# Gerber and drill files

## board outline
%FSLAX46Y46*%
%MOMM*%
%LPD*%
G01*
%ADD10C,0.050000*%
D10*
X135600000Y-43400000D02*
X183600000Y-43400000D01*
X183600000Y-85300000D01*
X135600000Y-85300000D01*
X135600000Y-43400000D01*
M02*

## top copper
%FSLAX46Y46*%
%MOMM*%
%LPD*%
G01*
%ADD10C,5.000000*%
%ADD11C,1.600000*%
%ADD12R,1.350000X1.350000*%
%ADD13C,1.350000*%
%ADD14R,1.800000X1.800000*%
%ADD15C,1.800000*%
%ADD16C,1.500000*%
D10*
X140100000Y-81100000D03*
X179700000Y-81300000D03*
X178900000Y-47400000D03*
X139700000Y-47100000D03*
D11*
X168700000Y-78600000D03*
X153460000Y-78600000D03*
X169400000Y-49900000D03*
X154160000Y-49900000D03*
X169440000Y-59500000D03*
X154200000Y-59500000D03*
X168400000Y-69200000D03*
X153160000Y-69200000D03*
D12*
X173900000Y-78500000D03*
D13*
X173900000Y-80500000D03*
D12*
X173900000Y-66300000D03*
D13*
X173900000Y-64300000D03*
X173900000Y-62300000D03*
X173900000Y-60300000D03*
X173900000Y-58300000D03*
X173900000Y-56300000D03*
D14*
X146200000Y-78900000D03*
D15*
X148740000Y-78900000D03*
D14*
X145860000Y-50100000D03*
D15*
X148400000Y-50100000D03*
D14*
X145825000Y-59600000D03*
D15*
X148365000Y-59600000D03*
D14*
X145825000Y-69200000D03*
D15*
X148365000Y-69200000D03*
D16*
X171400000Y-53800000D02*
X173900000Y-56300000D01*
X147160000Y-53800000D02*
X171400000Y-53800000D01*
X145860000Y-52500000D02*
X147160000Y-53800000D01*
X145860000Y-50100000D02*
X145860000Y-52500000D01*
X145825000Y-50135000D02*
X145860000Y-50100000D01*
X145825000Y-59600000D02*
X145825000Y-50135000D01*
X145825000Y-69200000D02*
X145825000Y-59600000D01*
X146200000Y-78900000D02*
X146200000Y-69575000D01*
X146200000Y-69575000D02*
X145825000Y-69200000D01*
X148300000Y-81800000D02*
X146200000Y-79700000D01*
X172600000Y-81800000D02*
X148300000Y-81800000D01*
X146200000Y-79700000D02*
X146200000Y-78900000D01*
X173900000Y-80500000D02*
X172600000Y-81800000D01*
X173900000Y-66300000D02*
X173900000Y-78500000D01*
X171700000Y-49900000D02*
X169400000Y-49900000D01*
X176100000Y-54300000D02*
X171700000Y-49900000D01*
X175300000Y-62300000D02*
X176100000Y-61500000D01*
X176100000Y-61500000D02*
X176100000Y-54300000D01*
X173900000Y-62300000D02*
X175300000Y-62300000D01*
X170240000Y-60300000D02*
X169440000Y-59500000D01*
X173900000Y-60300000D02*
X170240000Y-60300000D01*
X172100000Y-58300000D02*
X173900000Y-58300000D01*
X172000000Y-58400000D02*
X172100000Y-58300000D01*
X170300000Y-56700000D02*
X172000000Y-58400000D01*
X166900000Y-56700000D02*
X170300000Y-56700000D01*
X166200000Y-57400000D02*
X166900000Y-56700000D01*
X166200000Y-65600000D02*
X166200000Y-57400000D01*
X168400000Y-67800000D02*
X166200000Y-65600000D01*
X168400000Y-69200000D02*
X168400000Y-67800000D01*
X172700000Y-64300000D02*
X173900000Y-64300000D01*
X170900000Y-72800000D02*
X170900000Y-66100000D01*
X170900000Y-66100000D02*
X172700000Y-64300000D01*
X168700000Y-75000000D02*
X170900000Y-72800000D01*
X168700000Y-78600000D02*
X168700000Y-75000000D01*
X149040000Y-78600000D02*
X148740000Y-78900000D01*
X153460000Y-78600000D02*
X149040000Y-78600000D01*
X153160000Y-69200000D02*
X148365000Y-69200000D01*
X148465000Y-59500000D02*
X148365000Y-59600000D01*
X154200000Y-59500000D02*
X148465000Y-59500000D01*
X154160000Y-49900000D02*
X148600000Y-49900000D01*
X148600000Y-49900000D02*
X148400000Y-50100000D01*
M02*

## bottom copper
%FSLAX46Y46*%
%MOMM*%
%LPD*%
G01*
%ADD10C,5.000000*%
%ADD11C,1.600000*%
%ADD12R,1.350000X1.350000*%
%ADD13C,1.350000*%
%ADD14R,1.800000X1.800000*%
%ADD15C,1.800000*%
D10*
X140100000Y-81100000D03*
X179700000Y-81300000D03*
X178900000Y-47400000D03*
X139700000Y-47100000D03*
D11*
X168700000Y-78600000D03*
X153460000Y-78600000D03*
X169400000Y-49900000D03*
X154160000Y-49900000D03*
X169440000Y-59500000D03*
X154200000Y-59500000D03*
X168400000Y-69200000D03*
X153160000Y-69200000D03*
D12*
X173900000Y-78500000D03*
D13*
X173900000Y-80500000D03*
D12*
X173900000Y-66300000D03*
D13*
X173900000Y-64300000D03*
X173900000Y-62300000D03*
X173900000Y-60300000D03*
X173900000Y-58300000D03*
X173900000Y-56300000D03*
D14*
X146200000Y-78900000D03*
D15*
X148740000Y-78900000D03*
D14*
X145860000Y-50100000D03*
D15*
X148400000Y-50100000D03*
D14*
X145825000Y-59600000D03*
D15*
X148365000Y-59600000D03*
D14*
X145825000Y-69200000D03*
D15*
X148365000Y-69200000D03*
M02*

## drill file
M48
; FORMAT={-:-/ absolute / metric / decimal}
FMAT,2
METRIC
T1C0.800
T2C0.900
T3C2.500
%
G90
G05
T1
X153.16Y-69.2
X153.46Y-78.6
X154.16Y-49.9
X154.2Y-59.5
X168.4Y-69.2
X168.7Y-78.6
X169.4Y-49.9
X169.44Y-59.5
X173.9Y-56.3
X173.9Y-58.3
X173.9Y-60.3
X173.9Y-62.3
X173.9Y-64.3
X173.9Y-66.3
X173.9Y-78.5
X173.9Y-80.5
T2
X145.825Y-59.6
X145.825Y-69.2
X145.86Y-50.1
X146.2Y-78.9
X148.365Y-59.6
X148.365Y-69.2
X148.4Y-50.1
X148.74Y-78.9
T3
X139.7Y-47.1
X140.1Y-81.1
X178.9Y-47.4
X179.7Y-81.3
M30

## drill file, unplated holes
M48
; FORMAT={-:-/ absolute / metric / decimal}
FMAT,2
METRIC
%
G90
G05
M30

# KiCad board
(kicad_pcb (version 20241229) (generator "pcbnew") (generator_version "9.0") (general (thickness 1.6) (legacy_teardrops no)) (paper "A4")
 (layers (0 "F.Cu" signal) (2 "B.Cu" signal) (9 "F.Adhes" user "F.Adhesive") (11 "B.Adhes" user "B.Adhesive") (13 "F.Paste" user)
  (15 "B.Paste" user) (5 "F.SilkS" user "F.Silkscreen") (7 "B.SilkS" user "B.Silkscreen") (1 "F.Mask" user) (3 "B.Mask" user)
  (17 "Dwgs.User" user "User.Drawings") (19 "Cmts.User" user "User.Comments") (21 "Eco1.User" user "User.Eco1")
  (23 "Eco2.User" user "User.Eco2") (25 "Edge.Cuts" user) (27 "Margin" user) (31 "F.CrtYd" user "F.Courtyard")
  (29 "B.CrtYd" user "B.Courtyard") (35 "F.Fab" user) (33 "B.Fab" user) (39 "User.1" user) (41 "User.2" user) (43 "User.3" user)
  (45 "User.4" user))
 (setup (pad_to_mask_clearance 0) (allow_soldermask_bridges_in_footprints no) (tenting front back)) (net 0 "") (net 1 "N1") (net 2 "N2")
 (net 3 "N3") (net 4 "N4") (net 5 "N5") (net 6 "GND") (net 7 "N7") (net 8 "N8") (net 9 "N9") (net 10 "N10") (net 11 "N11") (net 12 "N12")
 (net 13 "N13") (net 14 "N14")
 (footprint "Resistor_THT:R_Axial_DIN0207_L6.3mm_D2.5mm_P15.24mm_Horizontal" (layer "F.Cu") (at 169.44 59.5 180)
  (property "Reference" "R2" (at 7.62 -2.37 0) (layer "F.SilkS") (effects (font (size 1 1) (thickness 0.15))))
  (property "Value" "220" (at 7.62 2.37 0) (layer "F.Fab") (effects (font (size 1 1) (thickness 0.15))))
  (pad "1" thru_hole circle (at 0 0 180) (size 1.6 1.6) (drill 0.8) (layers "*.Cu" "*.Mask") (remove_unused_layers no) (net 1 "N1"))
  (pad "2" thru_hole circle (at 15.24 0 180) (size 1.6 1.6) (drill 0.8) (layers "*.Cu" "*.Mask") (remove_unused_layers no) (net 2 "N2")))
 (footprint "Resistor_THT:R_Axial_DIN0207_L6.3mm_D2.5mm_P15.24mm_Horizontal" (layer "F.Cu") (at 168.7 78.6 180)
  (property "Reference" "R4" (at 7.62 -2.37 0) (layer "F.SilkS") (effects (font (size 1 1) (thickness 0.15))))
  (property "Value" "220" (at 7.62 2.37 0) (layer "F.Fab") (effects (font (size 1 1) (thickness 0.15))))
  (pad "1" thru_hole circle (at 0 0 180) (size 1.6 1.6) (drill 0.8) (layers "*.Cu" "*.Mask") (remove_unused_layers no) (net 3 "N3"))
  (pad "2" thru_hole circle (at 15.24 0 180) (size 1.6 1.6) (drill 0.8) (layers "*.Cu" "*.Mask") (remove_unused_layers no) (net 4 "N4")))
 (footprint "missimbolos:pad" (layer "F.Cu") (at 139.7 41.1)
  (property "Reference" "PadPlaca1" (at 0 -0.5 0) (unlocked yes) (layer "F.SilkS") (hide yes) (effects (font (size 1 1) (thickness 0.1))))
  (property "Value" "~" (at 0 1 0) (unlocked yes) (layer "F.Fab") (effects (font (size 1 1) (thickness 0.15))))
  (pad "1" thru_hole circle (at 0 6) (size 5 5) (drill 2.5) (layers "*.Cu" "*.Mask") (remove_unused_layers no) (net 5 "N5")))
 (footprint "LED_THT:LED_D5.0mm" (layer "F.Cu") (at 146.2 78.9)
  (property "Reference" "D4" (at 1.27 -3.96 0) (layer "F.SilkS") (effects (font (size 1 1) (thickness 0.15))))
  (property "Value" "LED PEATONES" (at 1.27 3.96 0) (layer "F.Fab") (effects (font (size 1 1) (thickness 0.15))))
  (pad "1" thru_hole rect (at 0 0) (size 1.8 1.8) (drill 0.9) (layers "*.Cu" "*.Mask") (remove_unused_layers no) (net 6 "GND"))
  (pad "2" thru_hole circle (at 2.54 0) (size 1.8 1.8) (drill 0.9) (layers "*.Cu" "*.Mask") (remove_unused_layers no) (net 4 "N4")))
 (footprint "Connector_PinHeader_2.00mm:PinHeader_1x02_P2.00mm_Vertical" (layer "F.Cu") (at 173.9 78.5)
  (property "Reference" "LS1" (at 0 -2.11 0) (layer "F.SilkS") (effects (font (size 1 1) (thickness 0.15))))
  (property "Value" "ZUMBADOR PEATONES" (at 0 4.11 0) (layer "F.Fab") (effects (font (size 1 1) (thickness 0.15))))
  (pad "1" thru_hole rect (at 0 0) (size 1.35 1.35) (drill 0.8) (layers "*.Cu" "*.Mask") (remove_unused_layers no) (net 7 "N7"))
  (pad "2" thru_hole circle (at 0 2) (size 1.35 1.35) (drill 0.8) (layers "*.Cu" "*.Mask") (remove_unused_layers no) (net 6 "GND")))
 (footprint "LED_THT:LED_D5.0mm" (layer "F.Cu") (at 145.825 69.2)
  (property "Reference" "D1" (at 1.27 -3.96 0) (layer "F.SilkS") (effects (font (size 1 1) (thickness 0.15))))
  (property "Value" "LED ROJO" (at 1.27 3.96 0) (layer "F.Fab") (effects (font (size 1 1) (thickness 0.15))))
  (pad "1" thru_hole rect (at 0 0) (size 1.8 1.8) (drill 0.9) (layers "*.Cu" "*.Mask") (remove_unused_layers no) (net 6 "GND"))
  (pad "2" thru_hole circle (at 2.54 0) (size 1.8 1.8) (drill 0.9) (layers "*.Cu" "*.Mask") (remove_unused_layers no) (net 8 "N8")))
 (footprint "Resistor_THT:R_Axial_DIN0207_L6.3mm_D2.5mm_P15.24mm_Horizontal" (layer "F.Cu") (at 169.4 49.9 180)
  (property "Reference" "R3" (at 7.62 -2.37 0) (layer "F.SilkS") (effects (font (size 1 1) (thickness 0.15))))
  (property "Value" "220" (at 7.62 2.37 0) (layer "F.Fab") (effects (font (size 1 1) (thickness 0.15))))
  (pad "1" thru_hole circle (at 0 0 180) (size 1.6 1.6) (drill 0.8) (layers "*.Cu" "*.Mask") (remove_unused_layers no) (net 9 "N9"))
  (pad "2" thru_hole circle (at 15.24 0 180) (size 1.6 1.6) (drill 0.8) (layers "*.Cu" "*.Mask") (remove_unused_layers no) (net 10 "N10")))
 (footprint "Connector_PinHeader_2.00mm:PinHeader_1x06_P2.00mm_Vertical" (layer "F.Cu") (at 173.9 66.3 180)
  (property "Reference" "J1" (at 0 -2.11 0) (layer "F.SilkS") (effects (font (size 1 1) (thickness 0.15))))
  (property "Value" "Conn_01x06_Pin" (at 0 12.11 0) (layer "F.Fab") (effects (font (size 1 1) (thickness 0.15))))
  (pad "1" thru_hole rect (at 0 0 180) (size 1.35 1.35) (drill 0.8) (layers "*.Cu" "*.Mask") (remove_unused_layers no) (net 7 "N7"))
  (pad "2" thru_hole circle (at 0 2 180) (size 1.35 1.35) (drill 0.8) (layers "*.Cu" "*.Mask") (remove_unused_layers no) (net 3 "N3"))
  (pad "3" thru_hole circle (at 0 4 180) (size 1.35 1.35) (drill 0.8) (layers "*.Cu" "*.Mask") (remove_unused_layers no) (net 9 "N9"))
  (pad "4" thru_hole circle (at 0 6 180) (size 1.35 1.35) (drill 0.8) (layers "*.Cu" "*.Mask") (remove_unused_layers no) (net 1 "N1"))
  (pad "5" thru_hole circle (at 0 8 180) (size 1.35 1.35) (drill 0.8) (layers "*.Cu" "*.Mask") (remove_unused_layers no) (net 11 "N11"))
  (pad "6" thru_hole circle (at 0 10 180) (size 1.35 1.35) (drill 0.8) (layers "*.Cu" "*.Mask") (remove_unused_layers no) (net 6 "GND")))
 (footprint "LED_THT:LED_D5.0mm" (layer "F.Cu") (at 145.825 59.6)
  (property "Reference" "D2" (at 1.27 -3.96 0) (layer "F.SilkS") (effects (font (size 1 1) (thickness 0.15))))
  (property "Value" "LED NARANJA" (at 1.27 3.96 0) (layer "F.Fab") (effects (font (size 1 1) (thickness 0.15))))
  (pad "1" thru_hole rect (at 0 0) (size 1.8 1.8) (drill 0.9) (layers "*.Cu" "*.Mask") (remove_unused_layers no) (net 6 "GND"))
  (pad "2" thru_hole circle (at 2.54 0) (size 1.8 1.8) (drill 0.9) (layers "*.Cu" "*.Mask") (remove_unused_layers no) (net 2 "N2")))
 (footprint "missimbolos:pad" (layer "F.Cu") (at 179.7 75.3)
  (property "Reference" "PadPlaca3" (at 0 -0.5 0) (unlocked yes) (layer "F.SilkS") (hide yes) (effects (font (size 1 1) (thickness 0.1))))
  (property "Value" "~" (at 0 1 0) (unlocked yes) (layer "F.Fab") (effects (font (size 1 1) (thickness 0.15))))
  (pad "1" thru_hole circle (at 0 6) (size 5 5) (drill 2.5) (layers "*.Cu" "*.Mask") (remove_unused_layers no) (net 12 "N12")))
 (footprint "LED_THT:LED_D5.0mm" (layer "F.Cu") (at 145.86 50.1)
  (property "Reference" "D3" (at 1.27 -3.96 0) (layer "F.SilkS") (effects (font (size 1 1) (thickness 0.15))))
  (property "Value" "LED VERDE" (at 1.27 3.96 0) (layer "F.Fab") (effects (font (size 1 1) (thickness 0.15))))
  (pad "1" thru_hole rect (at 0 0) (size 1.8 1.8) (drill 0.9) (layers "*.Cu" "*.Mask") (remove_unused_layers no) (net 6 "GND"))
  (pad "2" thru_hole circle (at 2.54 0) (size 1.8 1.8) (drill 0.9) (layers "*.Cu" "*.Mask") (remove_unused_layers no) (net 10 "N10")))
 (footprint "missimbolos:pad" (layer "F.Cu") (at 140.1 75.1)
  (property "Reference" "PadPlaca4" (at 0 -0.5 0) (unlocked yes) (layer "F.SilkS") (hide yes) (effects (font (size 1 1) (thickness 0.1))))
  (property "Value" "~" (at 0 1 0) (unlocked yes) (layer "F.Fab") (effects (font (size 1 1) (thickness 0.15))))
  (pad "1" thru_hole circle (at 0 6) (size 5 5) (drill 2.5) (layers "*.Cu" "*.Mask") (remove_unused_layers no) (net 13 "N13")))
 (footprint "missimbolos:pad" (layer "F.Cu") (at 178.9 41.4)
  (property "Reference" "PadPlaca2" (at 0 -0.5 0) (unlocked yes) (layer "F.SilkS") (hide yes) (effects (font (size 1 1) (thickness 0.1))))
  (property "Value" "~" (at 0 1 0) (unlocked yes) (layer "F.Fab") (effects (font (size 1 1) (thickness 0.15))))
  (pad "1" thru_hole circle (at 0 6) (size 5 5) (drill 2.5) (layers "*.Cu" "*.Mask") (remove_unused_layers no) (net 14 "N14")))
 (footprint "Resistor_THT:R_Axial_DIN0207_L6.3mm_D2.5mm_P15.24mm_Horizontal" (layer "F.Cu") (at 168.4 69.2 180)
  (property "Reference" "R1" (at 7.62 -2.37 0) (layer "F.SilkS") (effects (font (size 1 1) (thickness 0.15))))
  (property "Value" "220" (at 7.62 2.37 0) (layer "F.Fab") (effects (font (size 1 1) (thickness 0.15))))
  (pad "1" thru_hole circle (at 0 0 180) (size 1.6 1.6) (drill 0.8) (layers "*.Cu" "*.Mask") (remove_unused_layers no) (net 11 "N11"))
  (pad "2" thru_hole circle (at 15.24 0 180) (size 1.6 1.6) (drill 0.8) (layers "*.Cu" "*.Mask") (remove_unused_layers no) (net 8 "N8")))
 (gr_rect (start 135.6 43.4) (end 183.6 85.3) (stroke (width 0.05) (type default)) (fill no) (layer "Edge.Cuts"))
 (segment (start 146.2 79.7) (end 146.2 78.9) (width 1.5) (layer "F.Cu") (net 6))
 (segment (start 147.16 53.8) (end 171.4 53.8) (width 1.5) (layer "F.Cu") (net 6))
 (segment (start 146.2 69.575) (end 145.825 69.2) (width 1.5) (layer "F.Cu") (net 6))
 (segment (start 171.4 53.8) (end 173.9 56.3) (width 1.5) (layer "F.Cu") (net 6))
 (segment (start 173.9 80.5) (end 172.6 81.8) (width 1.5) (layer "F.Cu") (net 6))
 (segment (start 145.86 50.1) (end 145.86 52.5) (width 1.5) (layer "F.Cu") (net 6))
 (segment (start 145.825 69.2) (end 145.825 59.6) (width 1.5) (layer "F.Cu") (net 6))
 (segment (start 148.3 81.8) (end 146.2 79.7) (width 1.5) (layer "F.Cu") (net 6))
 (segment (start 145.86 52.5) (end 147.16 53.8) (width 1.5) (layer "F.Cu") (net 6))
 (segment (start 145.825 59.6) (end 145.825 50.135) (width 1.5) (layer "F.Cu") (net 6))
 (segment (start 172.6 81.8) (end 148.3 81.8) (width 1.5) (layer "F.Cu") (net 6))
 (segment (start 146.2 78.9) (end 146.2 69.575) (width 1.5) (layer "F.Cu") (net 6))
 (segment (start 145.825 50.135) (end 145.86 50.1) (width 1.5) (layer "F.Cu") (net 6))
 (segment (start 153.16 69.2) (end 148.365 69.2) (width 1.5) (layer "F.Cu") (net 8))
 (segment (start 154.2 59.5) (end 148.465 59.5) (width 1.5) (layer "F.Cu") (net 2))
 (segment (start 148.465 59.5) (end 148.365 59.6) (width 1.5) (layer "F.Cu") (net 2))
 (segment (start 154.16 49.9) (end 148.6 49.9) (width 1.5) (layer "F.Cu") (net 10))
 (segment (start 148.6 49.9) (end 148.4 50.1) (width 1.5) (layer "F.Cu") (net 10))
 (segment (start 153.46 78.6) (end 149.04 78.6) (width 1.5) (layer "F.Cu") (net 4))
 (segment (start 149.04 78.6) (end 148.74 78.9) (width 1.5) (layer "F.Cu") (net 4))
 (segment (start 168.7 75) (end 170.9 72.8) (width 1.5) (layer "F.Cu") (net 3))
 (segment (start 170.9 72.8) (end 170.9 66.1) (width 1.5) (layer "F.Cu") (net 3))
 (segment (start 168.7 78.6) (end 168.7 75) (width 1.5) (layer "F.Cu") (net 3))
 (segment (start 170.9 66.1) (end 172.7 64.3) (width 1.5) (layer "F.Cu") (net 3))
 (segment (start 172.7 64.3) (end 173.9 64.3) (width 1.5) (layer "F.Cu") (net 3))
 (segment (start 173.9 66.3) (end 173.9 78.5) (width 1.5) (layer "F.Cu") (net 7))
 (segment (start 172 58.4) (end 172.1 58.3) (width 1.5) (layer "F.Cu") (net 11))
 (segment (start 166.9 56.7) (end 170.3 56.7) (width 1.5) (layer "F.Cu") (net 11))
 (segment (start 168.4 67.8) (end 166.2 65.6) (width 1.5) (layer "F.Cu") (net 11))
 (segment (start 172.1 58.3) (end 173.9 58.3) (width 1.5) (layer "F.Cu") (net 11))
 (segment (start 166.2 65.6) (end 166.2 57.4) (width 1.5) (layer "F.Cu") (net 11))
 (segment (start 170.3 56.7) (end 172 58.4) (width 1.5) (layer "F.Cu") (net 11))
 (segment (start 168.4 69.2) (end 168.4 67.8) (width 1.5) (layer "F.Cu") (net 11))
 (segment (start 166.2 57.4) (end 166.9 56.7) (width 1.5) (layer "F.Cu") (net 11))
 (segment (start 176.1 61.5) (end 176.1 54.3) (width 1.5) (layer "F.Cu") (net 9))
 (segment (start 176.1 54.3) (end 171.7 49.9) (width 1.5) (layer "F.Cu") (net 9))
 (segment (start 173.9 62.3) (end 175.3 62.3) (width 1.5) (layer "F.Cu") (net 9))
 (segment (start 175.3 62.3) (end 176.1 61.5) (width 1.5) (layer "F.Cu") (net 9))
 (segment (start 171.7 49.9) (end 169.4 49.9) (width 1.5) (layer "F.Cu") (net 9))
 (segment (start 170.24 60.3) (end 169.44 59.5) (width 1.5) (layer "F.Cu") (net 1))
 (segment (start 173.9 60.3) (end 170.24 60.3) (width 1.5) (layer "F.Cu") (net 1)))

